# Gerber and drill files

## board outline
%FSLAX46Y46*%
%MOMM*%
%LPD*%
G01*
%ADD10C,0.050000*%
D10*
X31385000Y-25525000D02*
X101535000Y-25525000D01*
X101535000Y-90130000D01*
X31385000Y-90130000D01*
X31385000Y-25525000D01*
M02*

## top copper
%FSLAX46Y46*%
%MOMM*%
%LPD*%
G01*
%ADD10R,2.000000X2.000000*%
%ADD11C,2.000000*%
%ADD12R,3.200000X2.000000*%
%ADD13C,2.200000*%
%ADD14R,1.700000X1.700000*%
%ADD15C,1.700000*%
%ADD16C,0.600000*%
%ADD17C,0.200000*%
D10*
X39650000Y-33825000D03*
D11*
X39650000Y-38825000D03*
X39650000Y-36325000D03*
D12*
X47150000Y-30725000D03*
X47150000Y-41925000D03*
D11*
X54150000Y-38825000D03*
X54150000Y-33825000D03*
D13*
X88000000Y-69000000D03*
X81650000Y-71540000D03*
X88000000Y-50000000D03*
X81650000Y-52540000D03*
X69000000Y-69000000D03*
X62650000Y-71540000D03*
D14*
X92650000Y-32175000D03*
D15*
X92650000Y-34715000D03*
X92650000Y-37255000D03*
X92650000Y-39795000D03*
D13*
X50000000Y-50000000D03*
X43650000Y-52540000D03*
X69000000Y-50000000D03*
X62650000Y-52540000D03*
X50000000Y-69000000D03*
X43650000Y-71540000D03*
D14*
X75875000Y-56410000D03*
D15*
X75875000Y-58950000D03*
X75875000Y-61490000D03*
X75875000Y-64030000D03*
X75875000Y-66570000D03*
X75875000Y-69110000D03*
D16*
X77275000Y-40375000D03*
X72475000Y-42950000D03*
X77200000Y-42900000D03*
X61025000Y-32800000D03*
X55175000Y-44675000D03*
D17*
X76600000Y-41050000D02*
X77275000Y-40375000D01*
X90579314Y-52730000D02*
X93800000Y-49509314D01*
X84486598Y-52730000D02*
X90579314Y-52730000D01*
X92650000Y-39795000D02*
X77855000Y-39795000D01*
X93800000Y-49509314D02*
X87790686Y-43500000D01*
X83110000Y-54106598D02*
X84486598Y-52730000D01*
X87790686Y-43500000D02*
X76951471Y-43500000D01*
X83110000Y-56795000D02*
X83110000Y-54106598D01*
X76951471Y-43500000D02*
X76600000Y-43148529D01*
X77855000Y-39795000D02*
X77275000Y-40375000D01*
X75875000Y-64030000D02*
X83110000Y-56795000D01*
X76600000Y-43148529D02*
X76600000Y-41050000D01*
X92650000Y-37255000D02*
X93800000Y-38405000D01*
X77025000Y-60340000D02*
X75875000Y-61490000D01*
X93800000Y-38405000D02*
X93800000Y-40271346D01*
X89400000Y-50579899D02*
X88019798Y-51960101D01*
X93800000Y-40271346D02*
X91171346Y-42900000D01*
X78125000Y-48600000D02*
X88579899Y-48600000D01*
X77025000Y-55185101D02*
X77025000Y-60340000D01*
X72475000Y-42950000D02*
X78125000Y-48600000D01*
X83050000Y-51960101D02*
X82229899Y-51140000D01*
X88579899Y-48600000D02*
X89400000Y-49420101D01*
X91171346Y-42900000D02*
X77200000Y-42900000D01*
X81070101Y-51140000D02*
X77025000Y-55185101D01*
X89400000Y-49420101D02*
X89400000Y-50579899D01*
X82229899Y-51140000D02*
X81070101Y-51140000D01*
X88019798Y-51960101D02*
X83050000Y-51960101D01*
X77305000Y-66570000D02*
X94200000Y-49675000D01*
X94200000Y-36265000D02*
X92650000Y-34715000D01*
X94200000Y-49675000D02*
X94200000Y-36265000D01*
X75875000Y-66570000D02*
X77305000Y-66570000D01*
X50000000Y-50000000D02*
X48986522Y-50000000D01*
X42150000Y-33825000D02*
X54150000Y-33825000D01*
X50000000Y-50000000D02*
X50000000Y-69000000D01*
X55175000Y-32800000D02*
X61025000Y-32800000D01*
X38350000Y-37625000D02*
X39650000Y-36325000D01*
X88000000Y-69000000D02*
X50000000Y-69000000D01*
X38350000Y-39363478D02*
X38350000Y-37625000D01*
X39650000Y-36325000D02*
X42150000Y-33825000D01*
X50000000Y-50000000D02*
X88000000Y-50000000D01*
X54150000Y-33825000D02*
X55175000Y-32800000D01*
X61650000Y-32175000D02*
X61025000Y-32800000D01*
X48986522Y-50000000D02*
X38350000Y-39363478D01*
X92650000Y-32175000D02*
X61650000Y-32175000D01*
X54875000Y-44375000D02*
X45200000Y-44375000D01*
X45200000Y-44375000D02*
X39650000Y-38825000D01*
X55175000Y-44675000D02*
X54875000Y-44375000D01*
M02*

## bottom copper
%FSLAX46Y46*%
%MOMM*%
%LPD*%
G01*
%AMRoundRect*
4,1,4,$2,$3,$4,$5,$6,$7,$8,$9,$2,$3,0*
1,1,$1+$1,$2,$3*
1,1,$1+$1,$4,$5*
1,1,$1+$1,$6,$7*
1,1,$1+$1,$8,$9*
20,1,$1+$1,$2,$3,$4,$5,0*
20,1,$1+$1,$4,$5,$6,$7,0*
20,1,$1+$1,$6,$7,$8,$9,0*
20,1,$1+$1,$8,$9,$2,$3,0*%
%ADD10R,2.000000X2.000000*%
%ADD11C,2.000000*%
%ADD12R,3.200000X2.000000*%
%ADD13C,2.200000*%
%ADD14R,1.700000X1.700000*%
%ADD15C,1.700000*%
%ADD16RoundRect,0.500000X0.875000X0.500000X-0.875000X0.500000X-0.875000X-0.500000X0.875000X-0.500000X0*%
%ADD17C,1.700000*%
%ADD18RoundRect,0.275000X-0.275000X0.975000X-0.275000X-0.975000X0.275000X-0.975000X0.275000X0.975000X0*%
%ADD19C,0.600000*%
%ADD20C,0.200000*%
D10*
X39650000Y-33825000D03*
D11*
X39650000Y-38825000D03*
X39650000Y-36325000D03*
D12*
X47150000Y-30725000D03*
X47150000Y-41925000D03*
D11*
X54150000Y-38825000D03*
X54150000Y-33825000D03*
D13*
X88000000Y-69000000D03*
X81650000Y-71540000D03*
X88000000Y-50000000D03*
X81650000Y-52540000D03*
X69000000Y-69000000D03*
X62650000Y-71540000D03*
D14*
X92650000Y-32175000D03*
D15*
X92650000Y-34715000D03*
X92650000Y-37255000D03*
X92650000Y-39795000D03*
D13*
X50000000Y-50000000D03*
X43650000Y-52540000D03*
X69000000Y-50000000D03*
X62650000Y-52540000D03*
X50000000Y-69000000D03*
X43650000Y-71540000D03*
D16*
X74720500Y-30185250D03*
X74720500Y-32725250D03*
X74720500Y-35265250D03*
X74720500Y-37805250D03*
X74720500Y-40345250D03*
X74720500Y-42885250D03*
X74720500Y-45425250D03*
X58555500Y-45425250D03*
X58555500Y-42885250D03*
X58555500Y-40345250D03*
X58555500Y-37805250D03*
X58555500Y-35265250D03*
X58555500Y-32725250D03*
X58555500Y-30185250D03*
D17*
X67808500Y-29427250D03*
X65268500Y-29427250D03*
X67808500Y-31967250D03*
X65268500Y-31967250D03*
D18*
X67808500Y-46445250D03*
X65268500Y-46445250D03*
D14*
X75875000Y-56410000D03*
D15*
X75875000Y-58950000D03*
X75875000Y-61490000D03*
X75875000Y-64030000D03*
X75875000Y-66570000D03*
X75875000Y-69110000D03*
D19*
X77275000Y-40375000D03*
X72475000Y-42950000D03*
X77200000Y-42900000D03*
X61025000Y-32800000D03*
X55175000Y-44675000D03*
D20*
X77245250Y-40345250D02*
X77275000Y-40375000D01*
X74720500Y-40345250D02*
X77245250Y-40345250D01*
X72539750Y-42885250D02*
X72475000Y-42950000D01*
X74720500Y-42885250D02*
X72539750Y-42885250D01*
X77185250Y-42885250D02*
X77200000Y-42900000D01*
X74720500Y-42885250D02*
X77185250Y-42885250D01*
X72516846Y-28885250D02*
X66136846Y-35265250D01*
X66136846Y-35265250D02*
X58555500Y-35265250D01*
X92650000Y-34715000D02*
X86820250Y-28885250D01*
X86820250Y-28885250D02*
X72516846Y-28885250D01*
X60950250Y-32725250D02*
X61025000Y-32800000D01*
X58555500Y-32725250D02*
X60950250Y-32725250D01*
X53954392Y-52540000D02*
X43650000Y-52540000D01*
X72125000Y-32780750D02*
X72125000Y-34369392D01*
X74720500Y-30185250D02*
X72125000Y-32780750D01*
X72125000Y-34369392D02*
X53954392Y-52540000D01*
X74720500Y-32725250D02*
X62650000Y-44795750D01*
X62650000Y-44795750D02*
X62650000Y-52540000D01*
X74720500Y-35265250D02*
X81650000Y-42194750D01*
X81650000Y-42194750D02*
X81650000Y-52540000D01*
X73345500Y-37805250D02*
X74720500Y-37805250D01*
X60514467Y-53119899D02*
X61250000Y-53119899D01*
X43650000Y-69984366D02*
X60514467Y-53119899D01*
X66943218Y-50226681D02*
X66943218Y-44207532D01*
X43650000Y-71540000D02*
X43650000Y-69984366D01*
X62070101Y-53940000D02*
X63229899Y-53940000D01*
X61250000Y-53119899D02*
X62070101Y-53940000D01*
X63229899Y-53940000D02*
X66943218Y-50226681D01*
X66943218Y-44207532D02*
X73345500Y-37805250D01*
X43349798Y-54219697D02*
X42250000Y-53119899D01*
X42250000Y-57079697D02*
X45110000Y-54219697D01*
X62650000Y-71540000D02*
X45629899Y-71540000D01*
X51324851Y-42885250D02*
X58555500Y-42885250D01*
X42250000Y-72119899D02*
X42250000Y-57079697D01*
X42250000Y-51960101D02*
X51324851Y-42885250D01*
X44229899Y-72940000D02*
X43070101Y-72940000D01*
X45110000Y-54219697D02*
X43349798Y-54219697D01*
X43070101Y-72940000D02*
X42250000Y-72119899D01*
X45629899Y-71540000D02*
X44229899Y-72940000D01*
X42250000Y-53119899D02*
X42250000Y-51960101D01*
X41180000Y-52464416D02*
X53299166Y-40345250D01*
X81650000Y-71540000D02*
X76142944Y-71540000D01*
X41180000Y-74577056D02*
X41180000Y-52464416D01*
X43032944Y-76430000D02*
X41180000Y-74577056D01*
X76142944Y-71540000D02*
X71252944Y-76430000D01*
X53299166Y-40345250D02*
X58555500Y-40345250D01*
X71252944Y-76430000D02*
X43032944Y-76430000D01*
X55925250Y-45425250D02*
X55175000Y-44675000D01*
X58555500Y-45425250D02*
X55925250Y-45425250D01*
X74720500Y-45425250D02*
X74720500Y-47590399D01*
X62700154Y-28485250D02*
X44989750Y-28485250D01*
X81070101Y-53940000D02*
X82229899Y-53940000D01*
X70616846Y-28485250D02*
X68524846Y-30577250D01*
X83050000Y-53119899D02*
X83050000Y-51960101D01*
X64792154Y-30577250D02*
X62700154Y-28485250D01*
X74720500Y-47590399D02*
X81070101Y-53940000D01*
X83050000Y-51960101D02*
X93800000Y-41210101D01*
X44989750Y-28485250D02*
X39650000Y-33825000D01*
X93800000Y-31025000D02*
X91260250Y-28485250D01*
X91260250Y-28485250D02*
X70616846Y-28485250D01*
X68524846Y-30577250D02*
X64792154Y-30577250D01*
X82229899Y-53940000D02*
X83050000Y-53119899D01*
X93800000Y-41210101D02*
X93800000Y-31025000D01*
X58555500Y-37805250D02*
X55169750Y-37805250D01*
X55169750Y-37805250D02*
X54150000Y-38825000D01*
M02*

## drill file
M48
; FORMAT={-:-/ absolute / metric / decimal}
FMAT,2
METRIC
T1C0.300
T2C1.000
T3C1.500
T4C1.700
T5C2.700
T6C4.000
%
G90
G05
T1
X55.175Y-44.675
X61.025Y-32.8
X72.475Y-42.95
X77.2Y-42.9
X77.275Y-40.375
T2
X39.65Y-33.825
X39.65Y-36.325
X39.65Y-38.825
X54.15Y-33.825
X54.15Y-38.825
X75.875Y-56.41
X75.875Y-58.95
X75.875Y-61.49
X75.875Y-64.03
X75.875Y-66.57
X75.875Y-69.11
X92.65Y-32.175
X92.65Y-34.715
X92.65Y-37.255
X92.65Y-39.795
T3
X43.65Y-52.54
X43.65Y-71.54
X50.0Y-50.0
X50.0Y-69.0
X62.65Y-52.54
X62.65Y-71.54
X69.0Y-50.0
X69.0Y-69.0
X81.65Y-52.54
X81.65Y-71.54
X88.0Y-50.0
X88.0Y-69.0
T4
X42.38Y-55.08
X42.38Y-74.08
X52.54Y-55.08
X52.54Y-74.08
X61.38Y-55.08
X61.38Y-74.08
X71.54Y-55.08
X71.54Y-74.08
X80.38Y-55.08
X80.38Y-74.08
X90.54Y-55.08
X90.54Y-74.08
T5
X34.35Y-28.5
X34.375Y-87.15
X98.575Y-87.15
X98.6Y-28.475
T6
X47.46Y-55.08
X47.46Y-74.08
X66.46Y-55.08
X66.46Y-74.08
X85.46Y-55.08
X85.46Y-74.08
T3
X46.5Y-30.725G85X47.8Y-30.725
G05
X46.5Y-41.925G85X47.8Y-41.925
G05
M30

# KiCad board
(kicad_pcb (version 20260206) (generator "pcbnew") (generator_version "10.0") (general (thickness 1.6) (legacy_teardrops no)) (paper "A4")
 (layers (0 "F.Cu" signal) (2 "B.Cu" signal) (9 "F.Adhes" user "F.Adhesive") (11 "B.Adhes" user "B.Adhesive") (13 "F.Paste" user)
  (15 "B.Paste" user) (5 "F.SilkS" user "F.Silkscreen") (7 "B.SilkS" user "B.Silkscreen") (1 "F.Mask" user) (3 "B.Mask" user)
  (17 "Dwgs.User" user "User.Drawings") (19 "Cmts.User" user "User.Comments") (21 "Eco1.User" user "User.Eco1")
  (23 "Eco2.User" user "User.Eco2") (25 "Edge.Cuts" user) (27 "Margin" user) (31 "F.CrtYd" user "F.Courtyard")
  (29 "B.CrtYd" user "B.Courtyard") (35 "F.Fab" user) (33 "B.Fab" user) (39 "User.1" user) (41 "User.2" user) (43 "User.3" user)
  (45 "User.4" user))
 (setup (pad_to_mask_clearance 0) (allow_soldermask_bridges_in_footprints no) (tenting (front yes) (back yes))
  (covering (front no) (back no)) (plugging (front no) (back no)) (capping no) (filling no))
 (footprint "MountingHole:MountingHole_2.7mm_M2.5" (layer "F.Cu") (at 34.375 87.15)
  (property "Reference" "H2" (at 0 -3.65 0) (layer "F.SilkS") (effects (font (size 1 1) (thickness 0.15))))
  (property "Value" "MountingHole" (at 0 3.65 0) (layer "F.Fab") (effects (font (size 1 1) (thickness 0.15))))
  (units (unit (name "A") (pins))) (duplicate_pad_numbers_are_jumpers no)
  (pad "" np_thru_hole circle (at 0 0) (size 2.7 2.7) (drill 2.7) (layers "*.Cu" "*.Mask")))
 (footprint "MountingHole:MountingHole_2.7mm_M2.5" (layer "F.Cu") (at 98.575 87.15)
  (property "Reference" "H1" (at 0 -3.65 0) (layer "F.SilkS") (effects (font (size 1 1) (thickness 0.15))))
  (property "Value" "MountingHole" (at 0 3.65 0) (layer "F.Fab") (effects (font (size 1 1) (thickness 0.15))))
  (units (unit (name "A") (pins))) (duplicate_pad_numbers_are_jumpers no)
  (pad "" np_thru_hole circle (at 0 0) (size 2.7 2.7) (drill 2.7) (layers "*.Cu" "*.Mask")))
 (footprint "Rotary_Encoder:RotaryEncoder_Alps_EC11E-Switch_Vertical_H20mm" (layer "F.Cu") (at 39.65 33.825)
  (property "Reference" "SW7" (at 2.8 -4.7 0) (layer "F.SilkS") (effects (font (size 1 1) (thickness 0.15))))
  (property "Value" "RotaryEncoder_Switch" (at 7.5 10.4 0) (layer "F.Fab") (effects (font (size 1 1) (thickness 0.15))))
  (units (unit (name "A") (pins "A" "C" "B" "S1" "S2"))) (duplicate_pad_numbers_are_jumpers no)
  (pad "A" thru_hole rect (at 0 0) (size 2 2) (drill 1) (layers "*.Cu" "*.Mask") (remove_unused_layers no) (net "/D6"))
  (pad "B" thru_hole circle (at 0 5) (size 2 2) (drill 1) (layers "*.Cu" "*.Mask") (remove_unused_layers no) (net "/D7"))
  (pad "C" thru_hole circle (at 0 2.5) (size 2 2) (drill 1) (layers "*.Cu" "*.Mask") (remove_unused_layers no) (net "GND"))
  (pad "MP" thru_hole rect (at 7.5 -3.1) (size 3.2 2) (drill oval 2.8 1.5) (layers "*.Cu" "*.Mask") (remove_unused_layers no))
  (pad "MP" thru_hole rect (at 7.5 8.1) (size 3.2 2) (drill oval 2.8 1.5) (layers "*.Cu" "*.Mask") (remove_unused_layers no))
  (pad "S1" thru_hole circle (at 14.5 5) (size 2 2) (drill 1) (layers "*.Cu" "*.Mask") (remove_unused_layers no) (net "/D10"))
  (pad "S2" thru_hole circle (at 14.5 0) (size 2 2) (drill 1) (layers "*.Cu" "*.Mask") (remove_unused_layers no) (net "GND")))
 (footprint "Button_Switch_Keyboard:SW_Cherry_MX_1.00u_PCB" (layer "F.Cu") (at 88 69)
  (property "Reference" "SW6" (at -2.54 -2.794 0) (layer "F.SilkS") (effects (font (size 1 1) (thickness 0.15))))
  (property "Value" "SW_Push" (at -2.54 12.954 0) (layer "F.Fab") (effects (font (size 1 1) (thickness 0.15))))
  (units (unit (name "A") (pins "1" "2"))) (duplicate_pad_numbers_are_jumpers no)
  (pad "" np_thru_hole circle (at -7.62 5.08) (size 1.7 1.7) (drill 1.7) (layers "*.Cu" "*.Mask"))
  (pad "" np_thru_hole circle (at -2.54 5.08) (size 4 4) (drill 4) (layers "*.Cu" "*.Mask"))
  (pad "" np_thru_hole circle (at 2.54 5.08) (size 1.7 1.7) (drill 1.7) (layers "*.Cu" "*.Mask"))
  (pad "1" thru_hole circle (at 0 0) (size 2.2 2.2) (drill 1.5) (layers "*.Cu" "*.Mask") (remove_unused_layers no) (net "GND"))
  (pad "2" thru_hole circle (at -6.35 2.54) (size 2.2 2.2) (drill 1.5) (layers "*.Cu" "*.Mask") (remove_unused_layers no) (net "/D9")))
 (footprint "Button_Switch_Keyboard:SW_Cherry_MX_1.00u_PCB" (layer "F.Cu") (at 88 50)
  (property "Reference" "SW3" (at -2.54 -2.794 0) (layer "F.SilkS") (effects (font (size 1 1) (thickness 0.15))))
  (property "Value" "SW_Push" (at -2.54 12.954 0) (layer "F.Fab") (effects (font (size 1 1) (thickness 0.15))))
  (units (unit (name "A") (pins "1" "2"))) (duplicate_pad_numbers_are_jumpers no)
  (pad "" np_thru_hole circle (at -7.62 5.08) (size 1.7 1.7) (drill 1.7) (layers "*.Cu" "*.Mask"))
  (pad "" np_thru_hole circle (at -2.54 5.08) (size 4 4) (drill 4) (layers "*.Cu" "*.Mask"))
  (pad "" np_thru_hole circle (at 2.54 5.08) (size 1.7 1.7) (drill 1.7) (layers "*.Cu" "*.Mask"))
  (pad "1" thru_hole circle (at 0 0) (size 2.2 2.2) (drill 1.5) (layers "*.Cu" "*.Mask") (remove_unused_layers no) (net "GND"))
  (pad "2" thru_hole circle (at -6.35 2.54) (size 2.2 2.2) (drill 1.5) (layers "*.Cu" "*.Mask") (remove_unused_layers no) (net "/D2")))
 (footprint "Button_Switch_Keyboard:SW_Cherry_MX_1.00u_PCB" (layer "F.Cu") (at 69 69)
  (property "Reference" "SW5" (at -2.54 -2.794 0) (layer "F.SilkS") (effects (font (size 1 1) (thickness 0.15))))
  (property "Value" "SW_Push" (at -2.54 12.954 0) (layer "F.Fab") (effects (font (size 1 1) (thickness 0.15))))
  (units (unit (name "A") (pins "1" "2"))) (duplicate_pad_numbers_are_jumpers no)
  (pad "" np_thru_hole circle (at -7.62 5.08) (size 1.7 1.7) (drill 1.7) (layers "*.Cu" "*.Mask"))
  (pad "" np_thru_hole circle (at -2.54 5.08) (size 4 4) (drill 4) (layers "*.Cu" "*.Mask"))
  (pad "" np_thru_hole circle (at 2.54 5.08) (size 1.7 1.7) (drill 1.7) (layers "*.Cu" "*.Mask"))
  (pad "1" thru_hole circle (at 0 0) (size 2.2 2.2) (drill 1.5) (layers "*.Cu" "*.Mask") (remove_unused_layers no) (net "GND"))
  (pad "2" thru_hole circle (at -6.35 2.54) (size 2.2 2.2) (drill 1.5) (layers "*.Cu" "*.Mask") (remove_unused_layers no) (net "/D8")))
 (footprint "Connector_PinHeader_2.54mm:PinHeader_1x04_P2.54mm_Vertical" (layer "F.Cu") (at 92.65 32.175)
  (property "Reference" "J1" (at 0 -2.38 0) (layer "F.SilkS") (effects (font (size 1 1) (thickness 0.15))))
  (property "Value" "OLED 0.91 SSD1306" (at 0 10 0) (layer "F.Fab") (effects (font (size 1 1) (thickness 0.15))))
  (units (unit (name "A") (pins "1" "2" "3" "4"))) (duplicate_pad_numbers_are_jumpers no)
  (pad "1" thru_hole rect (at 0 0) (size 1.7 1.7) (drill 1) (layers "*.Cu" "*.Mask") (remove_unused_layers no) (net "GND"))
  (pad "2" thru_hole circle (at 0 2.54) (size 1.7 1.7) (drill 1) (layers "*.Cu" "*.Mask") (remove_unused_layers no) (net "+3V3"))
  (pad "3" thru_hole circle (at 0 5.08) (size 1.7 1.7) (drill 1) (layers "*.Cu" "*.Mask") (remove_unused_layers no) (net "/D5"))
  (pad "4" thru_hole circle (at 0 7.62) (size 1.7 1.7) (drill 1) (layers "*.Cu" "*.Mask") (remove_unused_layers no) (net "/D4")))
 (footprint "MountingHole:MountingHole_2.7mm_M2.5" (layer "F.Cu") (at 34.35 28.5)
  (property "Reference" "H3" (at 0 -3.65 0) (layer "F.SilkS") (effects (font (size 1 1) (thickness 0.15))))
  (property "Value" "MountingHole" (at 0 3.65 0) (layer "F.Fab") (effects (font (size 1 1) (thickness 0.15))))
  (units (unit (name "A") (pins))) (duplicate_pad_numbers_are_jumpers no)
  (pad "" np_thru_hole circle (at 0 0) (size 2.7 2.7) (drill 2.7) (layers "*.Cu" "*.Mask")))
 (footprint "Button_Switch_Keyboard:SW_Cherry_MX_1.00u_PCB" (layer "F.Cu") (at 50 50)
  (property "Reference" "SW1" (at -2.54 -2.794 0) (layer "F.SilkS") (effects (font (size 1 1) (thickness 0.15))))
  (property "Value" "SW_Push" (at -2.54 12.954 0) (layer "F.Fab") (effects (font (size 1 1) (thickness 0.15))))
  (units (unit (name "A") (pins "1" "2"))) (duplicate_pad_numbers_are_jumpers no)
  (pad "" np_thru_hole circle (at -7.62 5.08) (size 1.7 1.7) (drill 1.7) (layers "*.Cu" "*.Mask"))
  (pad "" np_thru_hole circle (at -2.54 5.08) (size 4 4) (drill 4) (layers "*.Cu" "*.Mask"))
  (pad "" np_thru_hole circle (at 2.54 5.08) (size 1.7 1.7) (drill 1.7) (layers "*.Cu" "*.Mask"))
  (pad "1" thru_hole circle (at 0 0) (size 2.2 2.2) (drill 1.5) (layers "*.Cu" "*.Mask") (remove_unused_layers no) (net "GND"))
  (pad "2" thru_hole circle (at -6.35 2.54) (size 2.2 2.2) (drill 1.5) (layers "*.Cu" "*.Mask") (remove_unused_layers no) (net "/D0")))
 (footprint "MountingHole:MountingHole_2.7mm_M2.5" (layer "F.Cu") (at 98.6 28.475)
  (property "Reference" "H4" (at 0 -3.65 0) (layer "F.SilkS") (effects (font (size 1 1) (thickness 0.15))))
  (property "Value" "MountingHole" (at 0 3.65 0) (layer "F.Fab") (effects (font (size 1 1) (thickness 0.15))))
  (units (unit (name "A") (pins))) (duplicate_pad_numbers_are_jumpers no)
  (pad "" np_thru_hole circle (at 0 0) (size 2.7 2.7) (drill 2.7) (layers "*.Cu" "*.Mask")))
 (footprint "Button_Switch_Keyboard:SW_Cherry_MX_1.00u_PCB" (layer "F.Cu") (at 69 50)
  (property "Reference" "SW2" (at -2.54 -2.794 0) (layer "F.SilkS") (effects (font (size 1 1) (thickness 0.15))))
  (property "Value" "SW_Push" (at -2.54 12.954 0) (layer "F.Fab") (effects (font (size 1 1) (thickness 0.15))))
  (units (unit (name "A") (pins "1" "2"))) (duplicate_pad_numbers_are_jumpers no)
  (pad "" np_thru_hole circle (at -7.62 5.08) (size 1.7 1.7) (drill 1.7) (layers "*.Cu" "*.Mask"))
  (pad "" np_thru_hole circle (at -2.54 5.08) (size 4 4) (drill 4) (layers "*.Cu" "*.Mask"))
  (pad "" np_thru_hole circle (at 2.54 5.08) (size 1.7 1.7) (drill 1.7) (layers "*.Cu" "*.Mask"))
  (pad "1" thru_hole circle (at 0 0) (size 2.2 2.2) (drill 1.5) (layers "*.Cu" "*.Mask") (remove_unused_layers no) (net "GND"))
  (pad "2" thru_hole circle (at -6.35 2.54) (size 2.2 2.2) (drill 1.5) (layers "*.Cu" "*.Mask") (remove_unused_layers no) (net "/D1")))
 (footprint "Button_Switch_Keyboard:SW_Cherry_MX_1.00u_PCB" (layer "F.Cu") (at 50 69)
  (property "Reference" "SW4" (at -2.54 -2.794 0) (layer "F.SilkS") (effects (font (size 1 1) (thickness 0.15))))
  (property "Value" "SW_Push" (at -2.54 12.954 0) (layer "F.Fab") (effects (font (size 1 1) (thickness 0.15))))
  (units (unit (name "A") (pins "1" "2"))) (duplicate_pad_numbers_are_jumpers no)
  (pad "" np_thru_hole circle (at -7.62 5.08) (size 1.7 1.7) (drill 1.7) (layers "*.Cu" "*.Mask"))
  (pad "" np_thru_hole circle (at -2.54 5.08) (size 4 4) (drill 4) (layers "*.Cu" "*.Mask"))
  (pad "" np_thru_hole circle (at 2.54 5.08) (size 1.7 1.7) (drill 1.7) (layers "*.Cu" "*.Mask"))
  (pad "1" thru_hole circle (at 0 0) (size 2.2 2.2) (drill 1.5) (layers "*.Cu" "*.Mask") (remove_unused_layers no) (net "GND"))
  (pad "2" thru_hole circle (at -6.35 2.54) (size 2.2 2.2) (drill 1.5) (layers "*.Cu" "*.Mask") (remove_unused_layers no) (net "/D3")))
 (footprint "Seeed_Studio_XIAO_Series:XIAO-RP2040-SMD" (layer "B.Cu") (at 75.5555 48.30525 180)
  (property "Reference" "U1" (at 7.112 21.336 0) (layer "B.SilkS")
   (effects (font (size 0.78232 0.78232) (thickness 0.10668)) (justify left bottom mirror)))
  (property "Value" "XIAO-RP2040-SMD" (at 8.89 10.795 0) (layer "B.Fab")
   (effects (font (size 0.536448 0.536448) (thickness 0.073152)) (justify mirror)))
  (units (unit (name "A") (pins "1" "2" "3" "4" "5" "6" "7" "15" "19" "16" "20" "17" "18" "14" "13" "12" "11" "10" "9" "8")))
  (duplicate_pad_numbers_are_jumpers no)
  (pad "1" smd roundrect (at 0.835 18.12 180) (size 2.75 2) (layers "B.Cu" "B.Mask" "B.Paste") (roundrect_rratio 0.25) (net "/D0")
   (solder_mask_margin 0.0508) (thermal_bridge_angle 45))
  (pad "2" smd roundrect (at 0.835 15.58 180) (size 2.75 2) (layers "B.Cu" "B.Mask" "B.Paste") (roundrect_rratio 0.25) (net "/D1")
   (solder_mask_margin 0.0508) (thermal_bridge_angle 45))
  (pad "3" smd roundrect (at 0.835 13.04 180) (size 2.75 2) (layers "B.Cu" "B.Mask" "B.Paste") (roundrect_rratio 0.25) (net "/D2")
   (solder_mask_margin 0.0508) (thermal_bridge_angle 45))
  (pad "4" smd roundrect (at 0.835 10.5 180) (size 2.75 2) (layers "B.Cu" "B.Mask" "B.Paste") (roundrect_rratio 0.25) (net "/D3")
   (solder_mask_margin 0.0508) (thermal_bridge_angle 45))
  (pad "5" smd roundrect (at 0.835 7.96 180) (size 2.75 2) (layers "B.Cu" "B.Mask" "B.Paste") (roundrect_rratio 0.25) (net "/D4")
   (solder_mask_margin 0.0508) (thermal_bridge_angle 45))
  (pad "6" smd roundrect (at 0.835 5.42 180) (size 2.75 2) (layers "B.Cu" "B.Mask" "B.Paste") (roundrect_rratio 0.25) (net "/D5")
   (solder_mask_margin 0.0508) (thermal_bridge_angle 45))
  (pad "7" smd roundrect (at 0.835 2.88 180) (size 2.75 2) (layers "B.Cu" "B.Mask" "B.Paste") (roundrect_rratio 0.25) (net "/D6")
   (solder_mask_margin 0.0508) (thermal_bridge_angle 45))
  (pad "8" smd roundrect (at 17 2.88 180) (size 2.75 2) (layers "B.Cu" "B.Mask" "B.Paste") (roundrect_rratio 0.25) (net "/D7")
   (solder_mask_margin 0.0508) (thermal_bridge_angle 45))
  (pad "9" smd roundrect (at 17 5.42 180) (size 2.75 2) (layers "B.Cu" "B.Mask" "B.Paste") (roundrect_rratio 0.25) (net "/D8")
   (solder_mask_margin 0.0508) (thermal_bridge_angle 45))
  (pad "10" smd roundrect (at 17 7.96 180) (size 2.75 2) (layers "B.Cu" "B.Mask" "B.Paste") (roundrect_rratio 0.25) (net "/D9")
   (solder_mask_margin 0.0508) (thermal_bridge_angle 45))
  (pad "11" smd roundrect (at 17 10.5 180) (size 2.75 2) (layers "B.Cu" "B.Mask" "B.Paste") (roundrect_rratio 0.25) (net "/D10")
   (solder_mask_margin 0.0508) (thermal_bridge_angle 45))
  (pad "12" smd roundrect (at 17 13.04 180) (size 2.75 2) (layers "B.Cu" "B.Mask" "B.Paste") (roundrect_rratio 0.25) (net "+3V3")
   (solder_mask_margin 0.0508) (thermal_bridge_angle 45))
  (pad "13" smd roundrect (at 17 15.58 180) (size 2.75 2) (layers "B.Cu" "B.Mask" "B.Paste") (roundrect_rratio 0.25) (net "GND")
   (solder_mask_margin 0.0508) (thermal_bridge_angle 45))
  (pad "14" smd roundrect (at 17 18.12 180) (size 2.75 2) (layers "B.Cu" "B.Mask" "B.Paste") (roundrect_rratio 0.25)
   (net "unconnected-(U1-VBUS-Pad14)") (solder_mask_margin 0.0508) (thermal_bridge_angle 45))
  (pad "15" smd circle (at 7.747 18.878 180) (size 1.7 1.7) (layers "B.Cu" "B.Mask" "B.Paste") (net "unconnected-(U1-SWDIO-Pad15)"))
  (pad "16" smd circle (at 10.287 18.878 180) (size 1.7 1.7) (layers "B.Cu" "B.Mask" "B.Paste") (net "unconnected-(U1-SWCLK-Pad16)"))
  (pad "17" smd circle (at 7.747 16.338 180) (size 1.7 1.7) (layers "B.Cu" "B.Mask" "B.Paste") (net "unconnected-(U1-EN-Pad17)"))
  (pad "18" smd circle (at 10.287 16.338 180) (size 1.7 1.7) (layers "B.Cu" "B.Mask" "B.Paste") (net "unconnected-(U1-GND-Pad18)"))
  (pad "19" smd roundrect (at 7.747 1.86 270) (size 2.5 1.1) (layers "B.Cu" "B.Mask" "B.Paste") (roundrect_rratio 0.25)
   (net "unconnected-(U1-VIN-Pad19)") (thermal_bridge_angle 45))
  (pad "20" smd roundrect (at 10.287 1.86 270) (size 2.5 1.1) (layers "B.Cu" "B.Mask" "B.Paste") (roundrect_rratio 0.25)
   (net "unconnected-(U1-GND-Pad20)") (thermal_bridge_angle 45)))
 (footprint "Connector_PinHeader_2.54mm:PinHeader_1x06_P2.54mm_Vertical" (layer "B.Cu") (at 75.875 56.41 180)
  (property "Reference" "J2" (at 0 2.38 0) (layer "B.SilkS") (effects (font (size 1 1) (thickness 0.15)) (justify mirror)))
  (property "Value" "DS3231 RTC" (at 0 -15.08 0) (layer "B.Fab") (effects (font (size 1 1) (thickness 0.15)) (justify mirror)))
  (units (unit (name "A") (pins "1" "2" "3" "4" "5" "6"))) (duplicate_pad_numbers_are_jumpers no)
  (pad "1" thru_hole rect (at 0 0 180) (size 1.7 1.7) (drill 1) (layers "*.Cu" "*.Mask") (remove_unused_layers no)
   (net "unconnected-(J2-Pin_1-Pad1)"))
  (pad "2" thru_hole circle (at 0 -2.54 180) (size 1.7 1.7) (drill 1) (layers "*.Cu" "*.Mask") (remove_unused_layers no)
   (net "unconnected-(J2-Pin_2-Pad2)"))
  (pad "3" thru_hole circle (at 0 -5.08 180) (size 1.7 1.7) (drill 1) (layers "*.Cu" "*.Mask") (remove_unused_layers no) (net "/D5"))
  (pad "4" thru_hole circle (at 0 -7.62 180) (size 1.7 1.7) (drill 1) (layers "*.Cu" "*.Mask") (remove_unused_layers no) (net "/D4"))
  (pad "5" thru_hole circle (at 0 -10.16 180) (size 1.7 1.7) (drill 1) (layers "*.Cu" "*.Mask") (remove_unused_layers no) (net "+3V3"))
  (pad "6" thru_hole circle (at 0 -12.7 180) (size 1.7 1.7) (drill 1) (layers "*.Cu" "*.Mask") (remove_unused_layers no) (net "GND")))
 (gr_rect (start 31.385 25.525) (end 101.535 90.13) (stroke (width 0.05) (type solid)) (fill no) (layer "Edge.Cuts"))
 (segment (start 76.6 41.05) (end 77.275 40.375) (width 0.2) (layer "F.Cu") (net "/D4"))
 (segment (start 90.579314 52.73) (end 93.8 49.509314) (width 0.2) (layer "F.Cu") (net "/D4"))
 (segment (start 84.486598 52.73) (end 90.579314 52.73) (width 0.2) (layer "F.Cu") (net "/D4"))
 (segment (start 92.65 39.795) (end 77.855 39.795) (width 0.2) (layer "F.Cu") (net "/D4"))
 (segment (start 93.8 49.509314) (end 87.790686 43.5) (width 0.2) (layer "F.Cu") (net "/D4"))
 (segment (start 83.11 54.106598) (end 84.486598 52.73) (width 0.2) (layer "F.Cu") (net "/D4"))
 (segment (start 87.790686 43.5) (end 76.951471 43.5) (width 0.2) (layer "F.Cu") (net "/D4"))
 (segment (start 83.11 56.795) (end 83.11 54.106598) (width 0.2) (layer "F.Cu") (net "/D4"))
 (segment (start 76.951471 43.5) (end 76.6 43.148529) (width 0.2) (layer "F.Cu") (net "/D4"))
 (segment (start 77.855 39.795) (end 77.275 40.375) (width 0.2) (layer "F.Cu") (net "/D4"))
 (segment (start 75.875 64.03) (end 83.11 56.795) (width 0.2) (layer "F.Cu") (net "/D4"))
 (segment (start 76.6 43.148529) (end 76.6 41.05) (width 0.2) (layer "F.Cu") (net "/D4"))
 (via (at 77.275 40.375) (size 0.6) (drill 0.3) (layers "F.Cu" "B.Cu") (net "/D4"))
 (segment (start 77.24525 40.34525) (end 77.275 40.375) (width 0.2) (layer "B.Cu") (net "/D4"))
 (segment (start 74.7205 40.34525) (end 77.24525 40.34525) (width 0.2) (layer "B.Cu") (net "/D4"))
 (segment (start 92.65 37.255) (end 93.8 38.405) (width 0.2) (layer "F.Cu") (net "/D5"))
 (segment (start 77.025 60.34) (end 75.875 61.49) (width 0.2) (layer "F.Cu") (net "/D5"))
 (segment (start 93.8 38.405) (end 93.8 40.271346) (width 0.2) (layer "F.Cu") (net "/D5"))
 (segment (start 89.4 50.579899) (end 88.019798 51.960101) (width 0.2) (layer "F.Cu") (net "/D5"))
 (segment (start 93.8 40.271346) (end 91.171346 42.9) (width 0.2) (layer "F.Cu") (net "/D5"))
 (segment (start 78.125 48.6) (end 88.579899 48.6) (width 0.2) (layer "F.Cu") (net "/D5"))
 (segment (start 77.025 55.185101) (end 77.025 60.34) (width 0.2) (layer "F.Cu") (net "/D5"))
 (segment (start 72.475 42.95) (end 78.125 48.6) (width 0.2) (layer "F.Cu") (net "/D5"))
 (segment (start 83.05 51.960101) (end 82.229899 51.14) (width 0.2) (layer "F.Cu") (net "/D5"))
 (segment (start 88.579899 48.6) (end 89.4 49.420101) (width 0.2) (layer "F.Cu") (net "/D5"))
 (segment (start 91.171346 42.9) (end 77.2 42.9) (width 0.2) (layer "F.Cu") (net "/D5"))
 (segment (start 81.070101 51.14) (end 77.025 55.185101) (width 0.2) (layer "F.Cu") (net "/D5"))
 (segment (start 89.4 49.420101) (end 89.4 50.579899) (width 0.2) (layer "F.Cu") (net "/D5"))
 (segment (start 82.229899 51.14) (end 81.070101 51.14) (width 0.2) (layer "F.Cu") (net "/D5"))
 (segment (start 88.019798 51.960101) (end 83.05 51.960101) (width 0.2) (layer "F.Cu") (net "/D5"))
 (via (at 72.475 42.95) (size 0.6) (drill 0.3) (layers "F.Cu" "B.Cu") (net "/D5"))
 (via (at 77.2 42.9) (size 0.6) (drill 0.3) (layers "F.Cu" "B.Cu") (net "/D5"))
 (segment (start 72.53975 42.88525) (end 72.475 42.95) (width 0.2) (layer "B.Cu") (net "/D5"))
 (segment (start 74.7205 42.88525) (end 72.53975 42.88525) (width 0.2) (layer "B.Cu") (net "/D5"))
 (segment (start 77.18525 42.88525) (end 77.2 42.9) (width 0.2) (layer "B.Cu") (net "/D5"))
 (segment (start 74.7205 42.88525) (end 77.18525 42.88525) (width 0.2) (layer "B.Cu") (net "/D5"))
 (segment (start 77.305 66.57) (end 94.2 49.675) (width 0.2) (layer "F.Cu") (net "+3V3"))
 (segment (start 94.2 36.265) (end 92.65 34.715) (width 0.2) (layer "F.Cu") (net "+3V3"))
 (segment (start 94.2 49.675) (end 94.2 36.265) (width 0.2) (layer "F.Cu") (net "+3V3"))
 (segment (start 75.875 66.57) (end 77.305 66.57) (width 0.2) (layer "F.Cu") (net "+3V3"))
 (segment (start 72.516846 28.88525) (end 66.136846 35.26525) (width 0.2) (layer "B.Cu") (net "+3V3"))
 (segment (start 66.136846 35.26525) (end 58.5555 35.26525) (width 0.2) (layer "B.Cu") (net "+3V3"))
 (segment (start 92.65 34.715) (end 86.82025 28.88525) (width 0.2) (layer "B.Cu") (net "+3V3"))
 (segment (start 86.82025 28.88525) (end 72.516846 28.88525) (width 0.2) (layer "B.Cu") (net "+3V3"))
 (segment (start 50 50) (end 48.986522 50) (width 0.2) (layer "F.Cu") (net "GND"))
 (segment (start 42.15 33.825) (end 54.15 33.825) (width 0.2) (layer "F.Cu") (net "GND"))
 (segment (start 50 50) (end 50 69) (width 0.2) (layer "F.Cu") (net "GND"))
 (segment (start 55.175 32.8) (end 61.025 32.8) (width 0.2) (layer "F.Cu") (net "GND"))
 (segment (start 38.35 37.625) (end 39.65 36.325) (width 0.2) (layer "F.Cu") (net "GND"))
 (segment (start 88 69) (end 50 69) (width 0.2) (layer "F.Cu") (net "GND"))
 (segment (start 38.35 39.363478) (end 38.35 37.625) (width 0.2) (layer "F.Cu") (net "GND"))
 (segment (start 39.65 36.325) (end 42.15 33.825) (width 0.2) (layer "F.Cu") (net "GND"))
 (segment (start 50 50) (end 88 50) (width 0.2) (layer "F.Cu") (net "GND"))
 (segment (start 54.15 33.825) (end 55.175 32.8) (width 0.2) (layer "F.Cu") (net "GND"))
 (segment (start 61.65 32.175) (end 61.025 32.8) (width 0.2) (layer "F.Cu") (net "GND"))
 (segment (start 48.986522 50) (end 38.35 39.363478) (width 0.2) (layer "F.Cu") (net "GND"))
 (segment (start 92.65 32.175) (end 61.65 32.175) (width 0.2) (layer "F.Cu") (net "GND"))
 (via (at 61.025 32.8) (size 0.6) (drill 0.3) (layers "F.Cu" "B.Cu") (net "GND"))
 (segment (start 60.95025 32.72525) (end 61.025 32.8) (width 0.2) (layer "B.Cu") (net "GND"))
 (segment (start 58.5555 32.72525) (end 60.95025 32.72525) (width 0.2) (layer "B.Cu") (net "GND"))
 (segment (start 53.954392 52.54) (end 43.65 52.54) (width 0.2) (layer "B.Cu") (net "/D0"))
 (segment (start 72.125 32.78075) (end 72.125 34.369392) (width 0.2) (layer "B.Cu") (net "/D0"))
 (segment (start 74.7205 30.18525) (end 72.125 32.78075) (width 0.2) (layer "B.Cu") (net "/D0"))
 (segment (start 72.125 34.369392) (end 53.954392 52.54) (width 0.2) (layer "B.Cu") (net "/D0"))
 (segment (start 74.7205 32.72525) (end 62.65 44.79575) (width 0.2) (layer "B.Cu") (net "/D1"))
 (segment (start 62.65 44.79575) (end 62.65 52.54) (width 0.2) (layer "B.Cu") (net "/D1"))
 (segment (start 74.7205 35.26525) (end 81.65 42.19475) (width 0.2) (layer "B.Cu") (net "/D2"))
 (segment (start 81.65 42.19475) (end 81.65 52.54) (width 0.2) (layer "B.Cu") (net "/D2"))
 (segment (start 73.3455 37.80525) (end 74.7205 37.80525) (width 0.2) (layer "B.Cu") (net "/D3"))
 (segment (start 60.514467 53.119899) (end 61.25 53.119899) (width 0.2) (layer "B.Cu") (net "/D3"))
 (segment (start 43.65 69.984366) (end 60.514467 53.119899) (width 0.2) (layer "B.Cu") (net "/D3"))
 (segment (start 66.943218 50.226681) (end 66.943218 44.207532) (width 0.2) (layer "B.Cu") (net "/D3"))
 (segment (start 43.65 71.54) (end 43.65 69.984366) (width 0.2) (layer "B.Cu") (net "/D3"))
 (segment (start 62.070101 53.94) (end 63.229899 53.94) (width 0.2) (layer "B.Cu") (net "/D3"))
 (segment (start 61.25 53.119899) (end 62.070101 53.94) (width 0.2) (layer "B.Cu") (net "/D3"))
 (segment (start 63.229899 53.94) (end 66.943218 50.226681) (width 0.2) (layer "B.Cu") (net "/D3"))
 (segment (start 66.943218 44.207532) (end 73.3455 37.80525) (width 0.2) (layer "B.Cu") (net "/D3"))
 (segment (start 43.349798 54.219697) (end 42.25 53.119899) (width 0.2) (layer "B.Cu") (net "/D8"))
 (segment (start 42.25 57.079697) (end 45.11 54.219697) (width 0.2) (layer "B.Cu") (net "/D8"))
 (segment (start 62.65 71.54) (end 45.629899 71.54) (width 0.2) (layer "B.Cu") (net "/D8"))
 (segment (start 51.324851 42.88525) (end 58.5555 42.88525) (width 0.2) (layer "B.Cu") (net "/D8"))
 (segment (start 42.25 72.119899) (end 42.25 57.079697) (width 0.2) (layer "B.Cu") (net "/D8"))
 (segment (start 42.25 51.960101) (end 51.324851 42.88525) (width 0.2) (layer "B.Cu") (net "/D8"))
 (segment (start 44.229899 72.94) (end 43.070101 72.94) (width 0.2) (layer "B.Cu") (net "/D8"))
 (segment (start 45.11 54.219697) (end 43.349798 54.219697) (width 0.2) (layer "B.Cu") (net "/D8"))
 (segment (start 43.070101 72.94) (end 42.25 72.119899) (width 0.2) (layer "B.Cu") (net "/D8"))
 (segment (start 45.629899 71.54) (end 44.229899 72.94) (width 0.2) (layer "B.Cu") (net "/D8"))
 (segment (start 42.25 53.119899) (end 42.25 51.960101) (width 0.2) (layer "B.Cu") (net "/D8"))
 (segment (start 41.18 52.464416) (end 53.299166 40.34525) (width 0.2) (layer "B.Cu") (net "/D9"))
 (segment (start 81.65 71.54) (end 76.142944 71.54) (width 0.2) (layer "B.Cu") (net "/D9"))
 (segment (start 41.18 74.577056) (end 41.18 52.464416) (width 0.2) (layer "B.Cu") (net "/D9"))
 (segment (start 43.032944 76.43) (end 41.18 74.577056) (width 0.2) (layer "B.Cu") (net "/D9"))
 (segment (start 76.142944 71.54) (end 71.252944 76.43) (width 0.2) (layer "B.Cu") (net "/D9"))
 (segment (start 53.299166 40.34525) (end 58.5555 40.34525) (width 0.2) (layer "B.Cu") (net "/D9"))
 (segment (start 71.252944 76.43) (end 43.032944 76.43) (width 0.2) (layer "B.Cu") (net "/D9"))
 (segment (start 54.875 44.375) (end 45.2 44.375) (width 0.2) (layer "F.Cu") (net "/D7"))
 (segment (start 45.2 44.375) (end 39.65 38.825) (width 0.2) (layer "F.Cu") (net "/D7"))
 (segment (start 55.175 44.675) (end 54.875 44.375) (width 0.2) (layer "F.Cu") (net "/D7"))
 (via (at 55.175 44.675) (size 0.6) (drill 0.3) (layers "F.Cu" "B.Cu") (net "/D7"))
 (segment (start 55.92525 45.42525) (end 55.175 44.675) (width 0.2) (layer "B.Cu") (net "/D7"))
 (segment (start 58.5555 45.42525) (end 55.92525 45.42525) (width 0.2) (layer "B.Cu") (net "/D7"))
 (segment (start 74.7205 45.42525) (end 74.7205 47.590399) (width 0.2) (layer "B.Cu") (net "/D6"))
 (segment (start 62.700154 28.48525) (end 44.98975 28.48525) (width 0.2) (layer "B.Cu") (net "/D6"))
 (segment (start 81.070101 53.94) (end 82.229899 53.94) (width 0.2) (layer "B.Cu") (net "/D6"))
 (segment (start 70.616846 28.48525) (end 68.524846 30.57725) (width 0.2) (layer "B.Cu") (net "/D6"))
 (segment (start 83.05 53.119899) (end 83.05 51.960101) (width 0.2) (layer "B.Cu") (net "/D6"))
 (segment (start 64.792154 30.57725) (end 62.700154 28.48525) (width 0.2) (layer "B.Cu") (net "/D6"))
 (segment (start 74.7205 47.590399) (end 81.070101 53.94) (width 0.2) (layer "B.Cu") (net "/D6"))
 (segment (start 83.05 51.960101) (end 93.8 41.210101) (width 0.2) (layer "B.Cu") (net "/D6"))
 (segment (start 44.98975 28.48525) (end 39.65 33.825) (width 0.2) (layer "B.Cu") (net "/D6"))
 (segment (start 93.8 31.025) (end 91.26025 28.48525) (width 0.2) (layer "B.Cu") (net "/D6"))
 (segment (start 91.26025 28.48525) (end 70.616846 28.48525) (width 0.2) (layer "B.Cu") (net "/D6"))
 (segment (start 68.524846 30.57725) (end 64.792154 30.57725) (width 0.2) (layer "B.Cu") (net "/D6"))
 (segment (start 82.229899 53.94) (end 83.05 53.119899) (width 0.2) (layer "B.Cu") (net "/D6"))
 (segment (start 93.8 41.210101) (end 93.8 31.025) (width 0.2) (layer "B.Cu") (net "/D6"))
 (segment (start 58.5555 37.80525) (end 55.16975 37.80525) (width 0.2) (layer "B.Cu") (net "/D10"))
 (segment (start 55.16975 37.80525) (end 54.15 38.825) (width 0.2) (layer "B.Cu") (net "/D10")))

